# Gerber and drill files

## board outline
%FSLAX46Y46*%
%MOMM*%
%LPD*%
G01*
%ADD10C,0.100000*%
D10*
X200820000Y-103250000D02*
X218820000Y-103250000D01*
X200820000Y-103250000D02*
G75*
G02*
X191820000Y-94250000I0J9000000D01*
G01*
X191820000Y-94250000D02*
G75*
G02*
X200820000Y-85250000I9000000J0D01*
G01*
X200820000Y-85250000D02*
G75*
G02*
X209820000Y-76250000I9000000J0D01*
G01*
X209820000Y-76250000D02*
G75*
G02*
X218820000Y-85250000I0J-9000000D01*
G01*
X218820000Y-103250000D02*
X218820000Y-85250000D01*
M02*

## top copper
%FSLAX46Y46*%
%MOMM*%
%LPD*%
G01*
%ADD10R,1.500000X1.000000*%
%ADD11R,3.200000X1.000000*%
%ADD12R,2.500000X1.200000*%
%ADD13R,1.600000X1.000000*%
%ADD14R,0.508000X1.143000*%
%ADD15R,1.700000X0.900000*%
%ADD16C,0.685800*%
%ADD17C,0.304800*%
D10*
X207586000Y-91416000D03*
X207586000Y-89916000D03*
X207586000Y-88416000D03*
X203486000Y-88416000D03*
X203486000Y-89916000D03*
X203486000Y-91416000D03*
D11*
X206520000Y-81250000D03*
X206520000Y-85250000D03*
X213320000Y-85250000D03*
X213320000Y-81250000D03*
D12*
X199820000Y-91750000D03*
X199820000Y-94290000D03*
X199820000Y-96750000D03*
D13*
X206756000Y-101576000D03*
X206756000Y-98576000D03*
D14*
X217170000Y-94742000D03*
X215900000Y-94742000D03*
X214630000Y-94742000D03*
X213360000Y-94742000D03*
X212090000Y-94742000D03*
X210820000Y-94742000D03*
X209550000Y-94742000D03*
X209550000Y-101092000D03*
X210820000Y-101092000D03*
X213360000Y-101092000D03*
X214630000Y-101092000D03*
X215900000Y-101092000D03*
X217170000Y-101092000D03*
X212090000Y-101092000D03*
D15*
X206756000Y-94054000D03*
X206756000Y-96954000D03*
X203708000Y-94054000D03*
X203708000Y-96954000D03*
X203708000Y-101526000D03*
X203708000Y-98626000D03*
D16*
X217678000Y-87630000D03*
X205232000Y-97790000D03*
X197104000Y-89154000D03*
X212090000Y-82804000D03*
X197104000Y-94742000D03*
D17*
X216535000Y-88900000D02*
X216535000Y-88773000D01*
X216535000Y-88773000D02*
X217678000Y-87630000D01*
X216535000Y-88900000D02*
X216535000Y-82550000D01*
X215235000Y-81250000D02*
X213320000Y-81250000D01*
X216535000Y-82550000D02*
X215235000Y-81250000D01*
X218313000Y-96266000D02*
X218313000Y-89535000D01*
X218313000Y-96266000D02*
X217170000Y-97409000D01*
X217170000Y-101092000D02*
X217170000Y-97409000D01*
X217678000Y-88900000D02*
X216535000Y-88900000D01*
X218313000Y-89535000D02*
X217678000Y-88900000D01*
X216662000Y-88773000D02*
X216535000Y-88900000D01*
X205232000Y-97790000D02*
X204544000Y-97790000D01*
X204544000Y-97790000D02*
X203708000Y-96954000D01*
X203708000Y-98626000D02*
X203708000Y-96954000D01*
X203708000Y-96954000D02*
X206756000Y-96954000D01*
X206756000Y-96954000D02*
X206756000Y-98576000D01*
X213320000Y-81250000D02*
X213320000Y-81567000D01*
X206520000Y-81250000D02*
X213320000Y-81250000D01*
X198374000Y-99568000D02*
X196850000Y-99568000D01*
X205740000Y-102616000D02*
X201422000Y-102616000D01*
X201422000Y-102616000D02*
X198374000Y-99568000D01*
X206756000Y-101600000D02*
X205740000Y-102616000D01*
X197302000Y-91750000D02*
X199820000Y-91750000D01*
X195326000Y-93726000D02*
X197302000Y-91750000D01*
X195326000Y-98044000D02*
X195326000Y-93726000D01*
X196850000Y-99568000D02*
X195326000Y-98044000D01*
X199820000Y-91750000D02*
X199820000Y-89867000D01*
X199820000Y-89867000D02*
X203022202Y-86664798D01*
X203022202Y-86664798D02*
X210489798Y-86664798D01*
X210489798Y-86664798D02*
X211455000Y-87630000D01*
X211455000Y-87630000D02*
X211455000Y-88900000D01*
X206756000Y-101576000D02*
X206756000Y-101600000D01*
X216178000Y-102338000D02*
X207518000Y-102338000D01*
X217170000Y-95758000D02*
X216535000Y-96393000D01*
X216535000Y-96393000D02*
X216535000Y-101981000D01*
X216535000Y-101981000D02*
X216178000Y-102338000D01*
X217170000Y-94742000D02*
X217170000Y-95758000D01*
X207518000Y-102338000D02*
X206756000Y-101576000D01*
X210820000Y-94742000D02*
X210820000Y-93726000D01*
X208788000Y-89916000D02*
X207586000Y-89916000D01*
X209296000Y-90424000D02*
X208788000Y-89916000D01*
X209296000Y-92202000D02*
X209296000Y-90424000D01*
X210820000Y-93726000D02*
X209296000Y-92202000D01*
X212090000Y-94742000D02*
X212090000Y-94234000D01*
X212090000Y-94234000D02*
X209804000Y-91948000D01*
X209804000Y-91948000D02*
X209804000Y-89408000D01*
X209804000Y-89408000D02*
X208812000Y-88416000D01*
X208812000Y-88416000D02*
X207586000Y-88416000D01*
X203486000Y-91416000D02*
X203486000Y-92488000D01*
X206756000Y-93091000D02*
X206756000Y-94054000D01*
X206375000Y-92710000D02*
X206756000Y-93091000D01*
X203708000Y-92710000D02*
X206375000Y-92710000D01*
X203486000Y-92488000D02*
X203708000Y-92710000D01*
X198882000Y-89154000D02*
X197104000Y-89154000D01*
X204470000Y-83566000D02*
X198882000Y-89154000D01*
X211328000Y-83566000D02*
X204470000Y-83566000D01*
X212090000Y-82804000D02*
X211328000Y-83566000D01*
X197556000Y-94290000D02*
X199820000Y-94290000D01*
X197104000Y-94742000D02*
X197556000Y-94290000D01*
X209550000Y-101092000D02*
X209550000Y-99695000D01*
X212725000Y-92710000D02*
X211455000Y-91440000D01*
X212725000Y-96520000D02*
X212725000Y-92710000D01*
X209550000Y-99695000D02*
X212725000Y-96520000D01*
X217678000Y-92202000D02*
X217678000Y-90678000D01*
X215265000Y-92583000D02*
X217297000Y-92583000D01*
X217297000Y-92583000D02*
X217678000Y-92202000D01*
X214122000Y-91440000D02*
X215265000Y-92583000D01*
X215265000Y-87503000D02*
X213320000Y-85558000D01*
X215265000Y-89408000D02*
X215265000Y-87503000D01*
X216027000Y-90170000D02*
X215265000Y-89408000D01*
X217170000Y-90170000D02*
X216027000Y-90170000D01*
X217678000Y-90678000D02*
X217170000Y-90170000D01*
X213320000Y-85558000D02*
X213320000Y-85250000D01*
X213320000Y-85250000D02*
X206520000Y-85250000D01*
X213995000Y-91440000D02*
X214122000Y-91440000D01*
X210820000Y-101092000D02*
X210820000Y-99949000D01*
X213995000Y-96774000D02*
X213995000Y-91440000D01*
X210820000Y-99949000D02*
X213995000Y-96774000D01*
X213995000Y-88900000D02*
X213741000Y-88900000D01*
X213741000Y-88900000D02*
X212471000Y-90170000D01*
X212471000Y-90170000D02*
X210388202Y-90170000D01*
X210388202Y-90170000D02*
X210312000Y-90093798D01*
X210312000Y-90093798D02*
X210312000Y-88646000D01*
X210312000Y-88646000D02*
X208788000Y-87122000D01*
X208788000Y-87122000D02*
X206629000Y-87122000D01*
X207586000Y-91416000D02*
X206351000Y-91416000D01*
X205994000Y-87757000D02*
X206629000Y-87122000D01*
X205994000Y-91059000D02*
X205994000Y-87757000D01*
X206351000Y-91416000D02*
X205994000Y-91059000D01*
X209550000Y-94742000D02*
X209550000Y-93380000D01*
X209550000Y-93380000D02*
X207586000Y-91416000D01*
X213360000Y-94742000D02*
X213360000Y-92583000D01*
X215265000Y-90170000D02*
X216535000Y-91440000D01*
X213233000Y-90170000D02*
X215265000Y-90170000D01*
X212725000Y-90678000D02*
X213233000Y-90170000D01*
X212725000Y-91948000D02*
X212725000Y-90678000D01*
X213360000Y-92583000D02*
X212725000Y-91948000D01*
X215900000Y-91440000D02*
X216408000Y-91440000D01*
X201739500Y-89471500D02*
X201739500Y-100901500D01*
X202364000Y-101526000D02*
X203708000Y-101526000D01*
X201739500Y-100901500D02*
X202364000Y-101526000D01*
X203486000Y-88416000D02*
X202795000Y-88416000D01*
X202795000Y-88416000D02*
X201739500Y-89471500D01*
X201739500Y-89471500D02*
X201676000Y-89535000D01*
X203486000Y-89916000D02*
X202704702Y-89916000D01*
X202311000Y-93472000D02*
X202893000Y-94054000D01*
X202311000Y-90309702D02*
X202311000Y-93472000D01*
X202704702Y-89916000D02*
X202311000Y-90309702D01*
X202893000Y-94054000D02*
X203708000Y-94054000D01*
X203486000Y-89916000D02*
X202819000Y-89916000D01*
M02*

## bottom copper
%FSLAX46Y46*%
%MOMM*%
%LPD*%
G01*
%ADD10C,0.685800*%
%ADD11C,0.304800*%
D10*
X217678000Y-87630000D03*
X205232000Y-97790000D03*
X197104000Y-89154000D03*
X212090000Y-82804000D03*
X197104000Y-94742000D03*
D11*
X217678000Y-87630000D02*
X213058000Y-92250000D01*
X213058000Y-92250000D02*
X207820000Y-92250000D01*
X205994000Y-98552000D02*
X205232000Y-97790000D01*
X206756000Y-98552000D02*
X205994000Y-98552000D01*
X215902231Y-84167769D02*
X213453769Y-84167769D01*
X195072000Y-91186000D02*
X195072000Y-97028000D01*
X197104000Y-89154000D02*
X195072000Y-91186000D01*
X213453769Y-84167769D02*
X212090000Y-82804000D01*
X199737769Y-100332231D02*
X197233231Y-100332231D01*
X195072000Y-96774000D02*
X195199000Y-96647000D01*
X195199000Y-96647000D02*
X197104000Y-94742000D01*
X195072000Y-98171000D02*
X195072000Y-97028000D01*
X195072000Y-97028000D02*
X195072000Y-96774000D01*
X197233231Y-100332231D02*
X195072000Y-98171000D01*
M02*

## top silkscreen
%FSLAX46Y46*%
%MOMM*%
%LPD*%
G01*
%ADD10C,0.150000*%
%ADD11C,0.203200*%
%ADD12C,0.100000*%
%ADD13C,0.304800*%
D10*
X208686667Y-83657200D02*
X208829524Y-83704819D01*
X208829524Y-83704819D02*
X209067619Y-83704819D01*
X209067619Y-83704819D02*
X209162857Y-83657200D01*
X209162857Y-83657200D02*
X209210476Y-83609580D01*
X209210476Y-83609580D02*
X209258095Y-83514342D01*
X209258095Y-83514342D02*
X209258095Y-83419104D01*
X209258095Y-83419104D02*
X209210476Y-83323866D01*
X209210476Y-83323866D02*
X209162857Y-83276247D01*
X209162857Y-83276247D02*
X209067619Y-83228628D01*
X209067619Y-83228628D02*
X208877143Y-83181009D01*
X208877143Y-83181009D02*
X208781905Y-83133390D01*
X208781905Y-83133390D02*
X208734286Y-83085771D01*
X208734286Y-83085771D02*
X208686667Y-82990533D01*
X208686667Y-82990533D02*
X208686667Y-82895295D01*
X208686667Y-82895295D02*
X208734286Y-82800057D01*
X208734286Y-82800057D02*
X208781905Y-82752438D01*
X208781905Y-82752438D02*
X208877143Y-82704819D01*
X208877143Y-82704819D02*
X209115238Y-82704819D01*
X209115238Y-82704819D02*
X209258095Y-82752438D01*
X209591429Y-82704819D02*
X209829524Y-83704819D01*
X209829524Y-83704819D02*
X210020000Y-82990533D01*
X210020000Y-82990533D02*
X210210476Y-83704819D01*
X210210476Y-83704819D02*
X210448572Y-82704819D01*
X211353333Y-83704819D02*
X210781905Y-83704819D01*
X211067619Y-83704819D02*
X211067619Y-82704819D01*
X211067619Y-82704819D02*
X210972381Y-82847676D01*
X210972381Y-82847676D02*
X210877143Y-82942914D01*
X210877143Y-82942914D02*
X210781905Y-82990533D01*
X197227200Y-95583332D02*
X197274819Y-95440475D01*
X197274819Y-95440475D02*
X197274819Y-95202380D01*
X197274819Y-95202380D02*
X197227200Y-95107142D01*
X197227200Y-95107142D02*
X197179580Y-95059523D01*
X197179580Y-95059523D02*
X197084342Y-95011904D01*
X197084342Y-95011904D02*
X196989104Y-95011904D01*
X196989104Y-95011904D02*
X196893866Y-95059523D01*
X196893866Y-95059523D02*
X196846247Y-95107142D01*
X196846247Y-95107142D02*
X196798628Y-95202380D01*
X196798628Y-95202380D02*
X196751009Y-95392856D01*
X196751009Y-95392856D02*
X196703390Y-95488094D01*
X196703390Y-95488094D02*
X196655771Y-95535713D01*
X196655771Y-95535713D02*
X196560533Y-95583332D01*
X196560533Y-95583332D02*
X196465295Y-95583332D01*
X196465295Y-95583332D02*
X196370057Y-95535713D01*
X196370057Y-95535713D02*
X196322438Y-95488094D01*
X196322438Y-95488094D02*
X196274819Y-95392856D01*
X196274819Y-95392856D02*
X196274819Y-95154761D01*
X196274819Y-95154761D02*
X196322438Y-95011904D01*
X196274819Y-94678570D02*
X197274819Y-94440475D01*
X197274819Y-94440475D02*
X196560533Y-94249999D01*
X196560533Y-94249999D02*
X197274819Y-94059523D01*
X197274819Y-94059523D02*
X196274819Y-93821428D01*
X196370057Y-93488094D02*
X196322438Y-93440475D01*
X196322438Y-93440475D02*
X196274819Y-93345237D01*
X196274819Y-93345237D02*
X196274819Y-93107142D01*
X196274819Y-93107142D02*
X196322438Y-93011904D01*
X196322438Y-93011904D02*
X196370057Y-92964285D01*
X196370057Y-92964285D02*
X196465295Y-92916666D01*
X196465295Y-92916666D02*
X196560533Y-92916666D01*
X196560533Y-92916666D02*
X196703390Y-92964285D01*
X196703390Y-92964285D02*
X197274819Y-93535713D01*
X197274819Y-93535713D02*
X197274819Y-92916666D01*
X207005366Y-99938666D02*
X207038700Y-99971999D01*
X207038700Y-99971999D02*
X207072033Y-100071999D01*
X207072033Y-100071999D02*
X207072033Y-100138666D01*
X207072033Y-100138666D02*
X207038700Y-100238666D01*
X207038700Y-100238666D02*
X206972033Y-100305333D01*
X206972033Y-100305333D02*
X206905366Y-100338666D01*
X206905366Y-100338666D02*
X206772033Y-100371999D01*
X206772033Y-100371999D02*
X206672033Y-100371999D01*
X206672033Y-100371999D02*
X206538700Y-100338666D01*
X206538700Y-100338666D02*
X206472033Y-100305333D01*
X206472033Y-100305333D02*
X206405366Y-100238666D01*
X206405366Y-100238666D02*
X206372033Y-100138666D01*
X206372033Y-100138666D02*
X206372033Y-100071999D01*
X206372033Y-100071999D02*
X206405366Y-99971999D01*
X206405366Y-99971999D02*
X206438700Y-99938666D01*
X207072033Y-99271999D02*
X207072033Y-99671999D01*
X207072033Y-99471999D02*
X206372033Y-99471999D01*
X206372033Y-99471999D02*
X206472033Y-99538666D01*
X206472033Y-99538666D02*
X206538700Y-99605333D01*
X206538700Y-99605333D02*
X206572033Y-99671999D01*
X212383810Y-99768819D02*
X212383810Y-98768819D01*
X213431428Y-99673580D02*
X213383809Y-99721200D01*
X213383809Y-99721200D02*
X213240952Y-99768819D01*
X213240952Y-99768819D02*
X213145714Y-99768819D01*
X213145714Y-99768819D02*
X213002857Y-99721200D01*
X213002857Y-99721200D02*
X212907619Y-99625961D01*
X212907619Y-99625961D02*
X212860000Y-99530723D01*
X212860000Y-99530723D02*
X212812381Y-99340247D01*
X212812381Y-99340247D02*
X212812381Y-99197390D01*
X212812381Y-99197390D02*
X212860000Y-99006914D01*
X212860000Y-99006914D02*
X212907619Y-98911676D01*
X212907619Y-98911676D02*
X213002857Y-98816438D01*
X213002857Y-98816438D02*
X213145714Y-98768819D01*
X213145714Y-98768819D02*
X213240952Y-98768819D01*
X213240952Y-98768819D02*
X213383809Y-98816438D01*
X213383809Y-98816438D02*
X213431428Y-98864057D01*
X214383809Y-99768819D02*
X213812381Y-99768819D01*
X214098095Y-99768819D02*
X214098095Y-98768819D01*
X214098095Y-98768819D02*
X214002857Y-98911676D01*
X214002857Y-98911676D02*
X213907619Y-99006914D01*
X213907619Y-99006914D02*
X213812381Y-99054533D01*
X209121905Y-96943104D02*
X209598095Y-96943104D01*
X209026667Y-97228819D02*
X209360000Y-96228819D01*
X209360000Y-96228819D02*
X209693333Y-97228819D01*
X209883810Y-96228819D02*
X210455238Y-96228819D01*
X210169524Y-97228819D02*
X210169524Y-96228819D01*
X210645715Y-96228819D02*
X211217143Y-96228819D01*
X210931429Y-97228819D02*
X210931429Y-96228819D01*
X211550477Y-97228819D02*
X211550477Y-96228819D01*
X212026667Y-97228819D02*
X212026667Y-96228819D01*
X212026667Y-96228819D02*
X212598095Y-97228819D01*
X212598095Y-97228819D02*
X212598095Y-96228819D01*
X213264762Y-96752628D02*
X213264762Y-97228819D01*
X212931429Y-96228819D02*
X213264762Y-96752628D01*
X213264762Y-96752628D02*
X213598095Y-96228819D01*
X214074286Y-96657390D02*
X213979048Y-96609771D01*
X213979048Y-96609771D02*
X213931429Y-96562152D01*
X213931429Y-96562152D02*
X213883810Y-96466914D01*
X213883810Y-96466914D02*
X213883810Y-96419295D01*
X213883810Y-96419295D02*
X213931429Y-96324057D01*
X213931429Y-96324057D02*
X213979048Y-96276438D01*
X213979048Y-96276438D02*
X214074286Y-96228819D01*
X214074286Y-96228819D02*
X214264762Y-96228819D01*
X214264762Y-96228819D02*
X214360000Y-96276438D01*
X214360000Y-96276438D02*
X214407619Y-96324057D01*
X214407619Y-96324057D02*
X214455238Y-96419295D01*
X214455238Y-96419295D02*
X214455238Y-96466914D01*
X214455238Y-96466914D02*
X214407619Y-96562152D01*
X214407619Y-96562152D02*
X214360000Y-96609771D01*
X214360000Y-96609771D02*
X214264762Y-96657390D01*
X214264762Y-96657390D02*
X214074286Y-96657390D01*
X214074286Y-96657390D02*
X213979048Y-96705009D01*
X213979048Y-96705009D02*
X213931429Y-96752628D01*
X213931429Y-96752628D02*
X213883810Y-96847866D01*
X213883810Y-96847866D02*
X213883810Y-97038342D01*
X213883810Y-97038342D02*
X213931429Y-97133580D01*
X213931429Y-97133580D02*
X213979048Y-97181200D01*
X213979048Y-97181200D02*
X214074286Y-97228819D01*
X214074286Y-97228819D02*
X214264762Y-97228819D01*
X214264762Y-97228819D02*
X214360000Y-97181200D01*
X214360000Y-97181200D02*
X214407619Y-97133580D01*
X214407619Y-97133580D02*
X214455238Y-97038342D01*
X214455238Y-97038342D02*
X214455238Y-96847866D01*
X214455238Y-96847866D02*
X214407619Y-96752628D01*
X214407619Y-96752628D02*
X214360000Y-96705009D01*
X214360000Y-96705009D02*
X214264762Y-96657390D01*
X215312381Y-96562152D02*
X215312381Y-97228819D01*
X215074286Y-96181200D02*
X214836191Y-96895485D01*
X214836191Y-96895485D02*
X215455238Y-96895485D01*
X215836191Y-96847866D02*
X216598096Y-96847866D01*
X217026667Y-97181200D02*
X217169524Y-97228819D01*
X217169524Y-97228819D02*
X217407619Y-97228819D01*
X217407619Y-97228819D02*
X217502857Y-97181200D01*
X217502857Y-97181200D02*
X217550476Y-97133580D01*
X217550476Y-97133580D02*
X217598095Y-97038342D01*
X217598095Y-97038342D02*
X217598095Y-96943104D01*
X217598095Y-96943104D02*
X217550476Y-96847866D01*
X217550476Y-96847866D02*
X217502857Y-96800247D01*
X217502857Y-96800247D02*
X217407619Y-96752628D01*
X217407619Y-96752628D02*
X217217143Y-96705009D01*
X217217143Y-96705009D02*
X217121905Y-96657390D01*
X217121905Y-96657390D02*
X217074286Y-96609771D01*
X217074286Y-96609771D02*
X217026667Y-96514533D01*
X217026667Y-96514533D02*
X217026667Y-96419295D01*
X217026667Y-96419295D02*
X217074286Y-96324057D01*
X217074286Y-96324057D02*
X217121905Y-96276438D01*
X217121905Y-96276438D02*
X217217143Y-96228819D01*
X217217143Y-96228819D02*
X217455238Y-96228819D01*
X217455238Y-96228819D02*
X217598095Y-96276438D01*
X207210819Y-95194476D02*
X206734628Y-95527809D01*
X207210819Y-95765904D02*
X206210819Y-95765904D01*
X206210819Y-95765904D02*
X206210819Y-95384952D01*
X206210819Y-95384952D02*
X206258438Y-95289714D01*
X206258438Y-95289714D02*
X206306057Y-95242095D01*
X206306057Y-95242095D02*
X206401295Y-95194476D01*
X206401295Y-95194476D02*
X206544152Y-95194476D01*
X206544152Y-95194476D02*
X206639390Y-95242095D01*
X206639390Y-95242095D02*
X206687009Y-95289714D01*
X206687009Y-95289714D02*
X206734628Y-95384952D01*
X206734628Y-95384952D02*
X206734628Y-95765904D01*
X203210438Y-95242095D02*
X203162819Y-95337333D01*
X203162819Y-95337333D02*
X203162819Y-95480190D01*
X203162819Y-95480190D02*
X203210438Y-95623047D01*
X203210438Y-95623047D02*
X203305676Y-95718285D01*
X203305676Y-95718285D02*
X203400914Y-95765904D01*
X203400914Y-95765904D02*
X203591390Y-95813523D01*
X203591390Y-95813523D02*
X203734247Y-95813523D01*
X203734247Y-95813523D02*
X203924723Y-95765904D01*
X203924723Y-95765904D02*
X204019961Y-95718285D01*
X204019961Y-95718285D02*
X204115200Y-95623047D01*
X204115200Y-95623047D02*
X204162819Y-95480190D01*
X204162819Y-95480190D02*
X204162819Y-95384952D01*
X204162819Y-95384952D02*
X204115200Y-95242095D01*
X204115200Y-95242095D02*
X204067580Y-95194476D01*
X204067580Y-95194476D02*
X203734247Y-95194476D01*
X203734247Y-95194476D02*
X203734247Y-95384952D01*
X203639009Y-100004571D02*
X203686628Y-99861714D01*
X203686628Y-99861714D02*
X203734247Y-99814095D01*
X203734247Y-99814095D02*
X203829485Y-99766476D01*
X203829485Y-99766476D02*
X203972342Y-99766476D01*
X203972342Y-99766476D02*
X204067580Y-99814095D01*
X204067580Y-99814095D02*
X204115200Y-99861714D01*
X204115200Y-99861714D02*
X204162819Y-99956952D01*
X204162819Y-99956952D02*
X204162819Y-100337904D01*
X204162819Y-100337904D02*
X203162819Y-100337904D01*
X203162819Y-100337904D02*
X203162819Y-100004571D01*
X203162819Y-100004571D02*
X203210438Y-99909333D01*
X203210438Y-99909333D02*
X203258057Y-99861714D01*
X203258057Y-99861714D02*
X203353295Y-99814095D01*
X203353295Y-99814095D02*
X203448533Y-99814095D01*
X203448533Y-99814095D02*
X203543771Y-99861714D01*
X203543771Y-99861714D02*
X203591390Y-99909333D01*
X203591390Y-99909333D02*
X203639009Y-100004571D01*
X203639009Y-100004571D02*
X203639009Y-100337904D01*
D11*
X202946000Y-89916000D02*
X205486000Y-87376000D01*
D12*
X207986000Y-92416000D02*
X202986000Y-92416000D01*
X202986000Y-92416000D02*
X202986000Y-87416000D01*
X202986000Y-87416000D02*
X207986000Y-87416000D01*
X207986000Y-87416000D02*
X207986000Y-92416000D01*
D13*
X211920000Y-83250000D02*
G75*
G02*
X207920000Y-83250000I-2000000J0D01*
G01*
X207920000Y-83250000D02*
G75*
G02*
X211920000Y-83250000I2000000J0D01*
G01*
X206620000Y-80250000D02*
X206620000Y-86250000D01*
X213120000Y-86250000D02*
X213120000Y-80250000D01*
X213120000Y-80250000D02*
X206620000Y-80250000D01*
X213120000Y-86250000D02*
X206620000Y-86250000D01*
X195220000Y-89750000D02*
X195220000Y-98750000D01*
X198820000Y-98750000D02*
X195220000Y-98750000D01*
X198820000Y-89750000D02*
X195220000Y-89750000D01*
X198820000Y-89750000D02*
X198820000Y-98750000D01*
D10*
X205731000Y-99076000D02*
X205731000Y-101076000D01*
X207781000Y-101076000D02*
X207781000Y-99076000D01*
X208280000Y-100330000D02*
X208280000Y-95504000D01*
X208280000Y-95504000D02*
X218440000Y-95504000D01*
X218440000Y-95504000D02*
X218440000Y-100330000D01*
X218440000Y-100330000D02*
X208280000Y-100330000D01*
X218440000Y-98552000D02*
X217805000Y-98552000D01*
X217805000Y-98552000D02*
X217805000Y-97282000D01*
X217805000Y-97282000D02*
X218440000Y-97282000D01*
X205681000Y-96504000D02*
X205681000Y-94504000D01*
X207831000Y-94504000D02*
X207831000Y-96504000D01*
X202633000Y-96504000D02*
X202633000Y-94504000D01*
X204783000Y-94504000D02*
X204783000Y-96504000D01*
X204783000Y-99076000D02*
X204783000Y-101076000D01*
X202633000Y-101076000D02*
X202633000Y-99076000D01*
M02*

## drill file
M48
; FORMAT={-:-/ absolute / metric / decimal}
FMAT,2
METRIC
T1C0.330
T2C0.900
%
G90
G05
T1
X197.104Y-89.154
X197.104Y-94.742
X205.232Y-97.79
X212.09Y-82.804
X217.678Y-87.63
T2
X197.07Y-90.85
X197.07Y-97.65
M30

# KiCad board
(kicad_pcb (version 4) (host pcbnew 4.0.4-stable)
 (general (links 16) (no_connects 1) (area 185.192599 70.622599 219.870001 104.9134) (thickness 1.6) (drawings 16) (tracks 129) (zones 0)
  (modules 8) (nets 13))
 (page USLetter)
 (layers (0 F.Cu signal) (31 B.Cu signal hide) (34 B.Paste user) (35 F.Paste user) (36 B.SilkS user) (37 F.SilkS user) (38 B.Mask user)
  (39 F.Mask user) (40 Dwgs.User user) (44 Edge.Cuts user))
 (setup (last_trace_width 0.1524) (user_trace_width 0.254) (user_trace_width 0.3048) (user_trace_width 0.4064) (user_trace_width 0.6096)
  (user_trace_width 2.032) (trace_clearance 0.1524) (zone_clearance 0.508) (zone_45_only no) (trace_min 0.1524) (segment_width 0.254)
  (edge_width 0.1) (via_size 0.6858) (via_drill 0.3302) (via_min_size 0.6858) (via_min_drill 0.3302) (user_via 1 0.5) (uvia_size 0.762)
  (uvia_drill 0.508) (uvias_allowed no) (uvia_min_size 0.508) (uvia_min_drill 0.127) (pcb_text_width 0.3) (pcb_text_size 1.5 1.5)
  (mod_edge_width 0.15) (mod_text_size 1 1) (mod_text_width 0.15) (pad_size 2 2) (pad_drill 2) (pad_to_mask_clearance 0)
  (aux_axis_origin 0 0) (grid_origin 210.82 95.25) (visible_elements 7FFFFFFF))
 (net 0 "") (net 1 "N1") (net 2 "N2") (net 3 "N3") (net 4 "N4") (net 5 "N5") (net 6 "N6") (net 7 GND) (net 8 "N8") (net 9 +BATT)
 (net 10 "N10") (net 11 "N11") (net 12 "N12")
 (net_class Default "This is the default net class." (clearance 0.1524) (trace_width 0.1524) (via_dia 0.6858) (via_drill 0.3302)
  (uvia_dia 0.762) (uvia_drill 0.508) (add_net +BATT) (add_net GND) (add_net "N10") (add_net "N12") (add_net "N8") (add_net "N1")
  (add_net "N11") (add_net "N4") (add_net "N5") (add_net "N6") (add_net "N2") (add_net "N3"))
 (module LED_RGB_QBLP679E (layer F.Cu) (at 205.486 89.916 180)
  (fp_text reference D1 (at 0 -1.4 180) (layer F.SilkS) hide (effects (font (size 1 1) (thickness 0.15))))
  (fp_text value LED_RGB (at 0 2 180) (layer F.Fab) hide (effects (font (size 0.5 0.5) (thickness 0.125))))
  (fp_line (start 2.54 0) (end 0 2.54) (layer F.SilkS) (width 0.2032))
  (fp_line (start -2.5 -2.5) (end 2.5 -2.5) (layer F.SilkS) (width 0.1))
  (fp_line (start 2.5 -2.5) (end 2.5 2.5) (layer F.SilkS) (width 0.1))
  (fp_line (start 2.5 2.5) (end -2.5 2.5) (layer F.SilkS) (width 0.1))
  (fp_line (start -2.5 2.5) (end -2.5 -2.5) (layer F.SilkS) (width 0.1))
  (pad 4 smd rect (at -2.1 -1.5 270) (size 1 1.5) (layers F.Cu F.Paste F.Mask) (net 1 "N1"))
  (pad 5 smd rect (at -2.1 0 270) (size 1 1.5) (layers F.Cu F.Paste F.Mask) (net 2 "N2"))
  (pad 6 smd rect (at -2.1 1.5 270) (size 1 1.5) (layers F.Cu F.Paste F.Mask) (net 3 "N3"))
  (pad 1 smd rect (at 2 1.5 270) (size 1 1.5) (layers F.Cu F.Paste F.Mask) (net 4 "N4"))
  (pad 2 smd rect (at 2 0 270) (size 1 1.5) (layers F.Cu F.Paste F.Mask) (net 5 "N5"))
  (pad 3 smd rect (at 2 -1.5 270) (size 1 1.5) (layers F.Cu F.Paste F.Mask) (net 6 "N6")))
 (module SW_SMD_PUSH (layer F.Cu) (at 213.32 85.25 180)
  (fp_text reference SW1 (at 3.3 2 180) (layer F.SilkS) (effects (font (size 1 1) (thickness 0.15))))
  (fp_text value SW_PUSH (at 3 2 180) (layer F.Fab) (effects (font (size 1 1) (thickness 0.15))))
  (fp_circle (center 3.4 2) (end 3.4 0) (layer F.SilkS) (width 0.3048))
  (fp_line (start 6.7 5) (end 6.7 -1) (layer F.SilkS) (width 0.3048))
  (fp_line (start 0.2 -1) (end 0.2 5) (layer F.SilkS) (width 0.3048))
  (fp_line (start 0.2 5) (end 6.7 5) (layer F.SilkS) (width 0.3048))
  (fp_line (start 0.2 -1) (end 6.7 -1) (layer F.SilkS) (width 0.3048))
  (pad 2 smd rect (at 6.8 4 180) (size 3.2 1) (layers F.Cu F.Paste F.Mask) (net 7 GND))
  (pad 1 smd rect (at 6.8 0 180) (size 3.2 1) (layers F.Cu F.Paste F.Mask) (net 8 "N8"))
  (pad 1 smd rect (at 0 0 180) (size 3.2 1) (layers F.Cu F.Paste F.Mask) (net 8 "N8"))
  (pad 2 smd rect (at 0 4 180) (size 3.2 1) (layers F.Cu F.Paste F.Mask) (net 7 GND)))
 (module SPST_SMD (layer F.Cu) (at 199.82 94.25 270)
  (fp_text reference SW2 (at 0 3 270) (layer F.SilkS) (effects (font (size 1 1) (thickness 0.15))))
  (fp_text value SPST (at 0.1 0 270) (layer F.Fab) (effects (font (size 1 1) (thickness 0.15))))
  (fp_line (start -4.5 4.6) (end 4.5 4.6) (layer F.SilkS) (width 0.3048))
  (fp_line (start 4.5 1) (end 4.5 4.6) (layer F.SilkS) (width 0.3048))
  (fp_line (start -4.5 1) (end -4.5 4.6) (layer F.SilkS) (width 0.3048))
  (fp_line (start -4.5 1) (end 4.5 1) (layer F.SilkS) (width 0.3048))
  (pad "" np_thru_hole circle (at 3.4 2.75 270) (size 0.9 0.9) (drill 0.9) (layers *.Cu *.Mask))
  (pad 1 smd rect (at -2.5 0 270) (size 1.2 2.5) (layers F.Cu F.Paste F.Mask) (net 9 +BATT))
  (pad 2 smd rect (at 0.04 0 270) (size 1.2 2.5) (layers F.Cu F.Paste F.Mask) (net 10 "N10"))
  (pad 3 smd rect (at 2.5 0 270) (size 1.2 2.5) (layers F.Cu F.Paste F.Mask))
  (pad "" np_thru_hole circle (at -3.4 2.75 270) (size 0.9 0.9) (drill 0.9) (layers *.Cu *.Mask)))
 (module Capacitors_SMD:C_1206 (layer F.Cu) (at 206.756 100.076 90)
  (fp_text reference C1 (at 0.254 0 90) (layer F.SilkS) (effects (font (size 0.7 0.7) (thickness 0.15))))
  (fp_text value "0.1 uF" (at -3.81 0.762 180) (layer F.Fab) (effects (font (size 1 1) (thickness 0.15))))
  (fp_line (start 1 -1.025) (end -1 -1.025) (layer F.SilkS) (width 0.15))
  (fp_line (start -1 1.025) (end 1 1.025) (layer F.SilkS) (width 0.15))
  (pad 1 smd rect (at -1.5 0 90) (size 1 1.6) (layers F.Cu F.Paste F.Mask) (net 9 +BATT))
  (pad 2 smd rect (at 1.5 0 90) (size 1 1.6) (layers F.Cu F.Paste F.Mask) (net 7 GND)))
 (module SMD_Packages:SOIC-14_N (layer F.Cu) (at 213.36 98.044 180)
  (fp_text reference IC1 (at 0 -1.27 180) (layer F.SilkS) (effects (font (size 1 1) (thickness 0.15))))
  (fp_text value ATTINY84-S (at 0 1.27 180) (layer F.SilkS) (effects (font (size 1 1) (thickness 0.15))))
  (fp_line (start 5.08 -2.286) (end 5.08 2.54) (layer F.SilkS) (width 0.15))
  (fp_line (start 5.08 2.54) (end -5.08 2.54) (layer F.SilkS) (width 0.15))
  (fp_line (start -5.08 2.54) (end -5.08 -2.286) (layer F.SilkS) (width 0.15))
  (fp_line (start -5.08 -2.286) (end 5.08 -2.286) (layer F.SilkS) (width 0.15))
  (fp_line (start -5.08 -0.508) (end -4.445 -0.508) (layer F.SilkS) (width 0.15))
  (fp_line (start -4.445 -0.508) (end -4.445 0.762) (layer F.SilkS) (width 0.15))
  (fp_line (start -4.445 0.762) (end -5.08 0.762) (layer F.SilkS) (width 0.15))
  (pad 1 smd rect (at -3.81 3.302 180) (size 0.508 1.143) (layers F.Cu F.Paste F.Mask) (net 9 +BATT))
  (pad 2 smd rect (at -2.54 3.302 180) (size 0.508 1.143) (layers F.Cu F.Paste F.Mask))
  (pad 3 smd rect (at -1.27 3.302 180) (size 0.508 1.143) (layers F.Cu F.Paste F.Mask))
  (pad 4 smd rect (at 0 3.302 180) (size 0.508 1.143) (layers F.Cu F.Paste F.Mask) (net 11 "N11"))
  (pad 5 smd rect (at 1.27 3.302 180) (size 0.508 1.143) (layers F.Cu F.Paste F.Mask) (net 3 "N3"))
  (pad 6 smd rect (at 2.54 3.302 180) (size 0.508 1.143) (layers F.Cu F.Paste F.Mask) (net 2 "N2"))
  (pad 7 smd rect (at 3.81 3.302 180) (size 0.508 1.143) (layers F.Cu F.Paste F.Mask) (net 1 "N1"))
  (pad 8 smd rect (at 3.81 -3.048 180) (size 0.508 1.143) (layers F.Cu F.Paste F.Mask) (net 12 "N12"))
  (pad 9 smd rect (at 2.54 -3.048 180) (size 0.508 1.143) (layers F.Cu F.Paste F.Mask) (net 8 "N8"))
  (pad 11 smd rect (at 0 -3.048 180) (size 0.508 1.143) (layers F.Cu F.Paste F.Mask))
  (pad 12 smd rect (at -1.27 -3.048 180) (size 0.508 1.143) (layers F.Cu F.Paste F.Mask))
  (pad 13 smd rect (at -2.54 -3.048 180) (size 0.508 1.143) (layers F.Cu F.Paste F.Mask))
  (pad 14 smd rect (at -3.81 -3.048 180) (size 0.508 1.143) (layers F.Cu F.Paste F.Mask) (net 7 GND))
  (pad 10 smd rect (at 1.27 -3.048 180) (size 0.508 1.143) (layers F.Cu F.Paste F.Mask)))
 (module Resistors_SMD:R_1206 (layer F.Cu) (at 206.756 95.504 270)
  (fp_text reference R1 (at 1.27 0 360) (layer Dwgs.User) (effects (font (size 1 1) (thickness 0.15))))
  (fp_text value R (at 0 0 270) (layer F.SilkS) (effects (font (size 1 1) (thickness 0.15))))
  (fp_line (start 1 1.075) (end -1 1.075) (layer F.SilkS) (width 0.15))
  (fp_line (start -1 -1.075) (end 1 -1.075) (layer F.SilkS) (width 0.15))
  (pad 1 smd rect (at -1.45 0 270) (size 0.9 1.7) (layers F.Cu F.Paste F.Mask) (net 6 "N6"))
  (pad 2 smd rect (at 1.45 0 270) (size 0.9 1.7) (layers F.Cu F.Paste F.Mask) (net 7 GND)))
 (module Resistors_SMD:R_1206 (layer F.Cu) (at 203.708 95.504 270)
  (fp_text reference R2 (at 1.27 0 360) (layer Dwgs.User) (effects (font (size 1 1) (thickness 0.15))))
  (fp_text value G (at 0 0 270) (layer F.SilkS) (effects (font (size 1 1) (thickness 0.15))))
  (fp_line (start 1 1.075) (end -1 1.075) (layer F.SilkS) (width 0.15))
  (fp_line (start -1 -1.075) (end 1 -1.075) (layer F.SilkS) (width 0.15))
  (pad 1 smd rect (at -1.45 0 270) (size 0.9 1.7) (layers F.Cu F.Paste F.Mask) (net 5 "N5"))
  (pad 2 smd rect (at 1.45 0 270) (size 0.9 1.7) (layers F.Cu F.Paste F.Mask) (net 7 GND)))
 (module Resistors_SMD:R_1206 (layer F.Cu) (at 203.708 100.076 90)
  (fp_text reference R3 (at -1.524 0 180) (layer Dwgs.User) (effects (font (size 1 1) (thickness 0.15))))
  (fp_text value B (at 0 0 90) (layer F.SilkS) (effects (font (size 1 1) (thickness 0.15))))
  (fp_line (start 1 1.075) (end -1 1.075) (layer F.SilkS) (width 0.15))
  (fp_line (start -1 -1.075) (end 1 -1.075) (layer F.SilkS) (width 0.15))
  (pad 1 smd rect (at -1.45 0 90) (size 0.9 1.7) (layers F.Cu F.Paste F.Mask) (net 4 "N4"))
  (pad 2 smd rect (at 1.45 0 90) (size 0.9 1.7) (layers F.Cu F.Paste F.Mask) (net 7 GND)))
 (gr_line (start 200.82 103.25) (end 218.82 103.25) (angle 90) (layer Edge.Cuts) (width 0.1))
 (gr_arc (start 200.82 94.25) (end 200.82 103.25) (angle 90) (layer Edge.Cuts) (width 0.1))
 (gr_arc (start 200.82 94.25) (end 191.82 94.25) (angle 90) (layer Edge.Cuts) (width 0.1))
 (gr_arc (start 209.82 85.25) (end 200.82 85.25) (angle 90) (layer Edge.Cuts) (width 0.1))
 (gr_arc (start 209.82 85.25) (end 209.82 76.25) (angle 90) (layer Edge.Cuts) (width 0.1))
 (gr_line (start 218.82 103.25) (end 218.82 85.25) (angle 90) (layer Edge.Cuts) (width 0.1))
 (segment (start 216.535 88.9) (end 216.535 88.773) (width 0.3048) (layer F.Cu) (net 7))
 (segment (start 216.535 88.773) (end 217.678 87.63) (width 0.3048) (layer F.Cu) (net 7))
 (segment (start 217.678 87.63) (end 213.058 92.25) (width 0.3048) (layer B.Cu) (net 7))
 (via (at 217.678 87.63) (size 0.6858) (drill 0.3302) (layers F.Cu B.Cu) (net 7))
 (segment (start 213.058 92.25) (end 207.82 92.25) (width 0.3048) (layer B.Cu) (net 7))
 (segment (start 216.535 88.9) (end 216.535 82.55) (width 0.3048) (layer F.Cu) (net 7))
 (segment (start 215.235 81.25) (end 213.32 81.25) (width 0.3048) (layer F.Cu) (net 7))
 (segment (start 216.535 82.55) (end 215.235 81.25) (width 0.3048) (layer F.Cu) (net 7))
 (segment (start 218.313 96.266) (end 218.313 89.535) (width 0.3048) (layer F.Cu) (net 7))
 (segment (start 218.313 96.266) (end 217.17 97.409) (width 0.3048) (layer F.Cu) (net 7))
 (segment (start 217.17 101.092) (end 217.17 97.409) (width 0.3048) (layer F.Cu) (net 7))
 (segment (start 217.678 88.9) (end 216.535 88.9) (width 0.3048) (layer F.Cu) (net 7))
 (segment (start 218.313 89.535) (end 217.678 88.9) (width 0.3048) (layer F.Cu) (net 7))
 (segment (start 216.662 88.773) (end 216.535 88.9) (width 0.3048) (layer F.Cu) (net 7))
 (segment (start 205.232 97.79) (end 204.544 97.79) (width 0.3048) (layer F.Cu) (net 7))
 (segment (start 205.994 98.552) (end 205.232 97.79) (width 0.3048) (layer B.Cu) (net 7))
 (via (at 205.232 97.79) (size 0.6858) (drill 0.3302) (layers F.Cu B.Cu) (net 7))
 (segment (start 204.544 97.79) (end 203.708 96.954) (width 0.3048) (layer F.Cu) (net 7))
 (segment (start 206.756 98.552) (end 205.994 98.552) (width 0.3048) (layer B.Cu) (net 7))
 (segment (start 203.708 98.626) (end 203.708 96.954) (width 0.3048) (layer F.Cu) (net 7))
 (segment (start 203.708 96.954) (end 206.756 96.954) (width 0.3048) (layer F.Cu) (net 7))
 (segment (start 206.756 96.954) (end 206.756 98.576) (width 0.3048) (layer F.Cu) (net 7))
 (segment (start 213.32 81.25) (end 213.32 81.567) (width 0.3048) (layer F.Cu) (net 7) (status 30))
 (segment (start 206.52 81.25) (end 213.32 81.25) (width 0.3048) (layer F.Cu) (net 7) (status 30))
 (segment (start 198.374 99.568) (end 196.85 99.568) (width 0.3048) (layer F.Cu) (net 9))
 (segment (start 205.74 102.616) (end 201.422 102.616) (width 0.3048) (layer F.Cu) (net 9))
 (segment (start 201.422 102.616) (end 198.374 99.568) (width 0.3048) (layer F.Cu) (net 9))
 (segment (start 206.756 101.6) (end 205.74 102.616) (width 0.3048) (layer F.Cu) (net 9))
 (segment (start 197.302 91.75) (end 199.82 91.75) (width 0.3048) (layer F.Cu) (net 9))
 (segment (start 195.326 93.726) (end 197.302 91.75) (width 0.3048) (layer F.Cu) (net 9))
 (segment (start 195.326 98.044) (end 195.326 93.726) (width 0.3048) (layer F.Cu) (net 9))
 (segment (start 196.85 99.568) (end 195.326 98.044) (width 0.3048) (layer F.Cu) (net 9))
 (segment (start 199.82 91.75) (end 199.82 89.867) (width 0.3048) (layer F.Cu) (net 9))
 (segment (start 199.82 89.867) (end 203.022202 86.664798) (width 0.3048) (layer F.Cu) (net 9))
 (segment (start 203.022202 86.664798) (end 210.489798 86.664798) (width 0.3048) (layer F.Cu) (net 9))
 (segment (start 210.489798 86.664798) (end 211.455 87.63) (width 0.3048) (layer F.Cu) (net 9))
 (segment (start 211.455 87.63) (end 211.455 88.9) (width 0.3048) (layer F.Cu) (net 9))
 (segment (start 206.756 101.576) (end 206.756 101.6) (width 0.3048) (layer F.Cu) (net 9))
 (segment (start 216.178 102.338) (end 207.518 102.338) (width 0.3048) (layer F.Cu) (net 9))
 (segment (start 217.17 95.758) (end 216.535 96.393) (width 0.3048) (layer F.Cu) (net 9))
 (segment (start 216.535 96.393) (end 216.535 101.981) (width 0.3048) (layer F.Cu) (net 9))
 (segment (start 216.535 101.981) (end 216.178 102.338) (width 0.3048) (layer F.Cu) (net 9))
 (segment (start 217.17 94.742) (end 217.17 95.758) (width 0.3048) (layer F.Cu) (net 9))
 (segment (start 207.518 102.338) (end 206.756 101.576) (width 0.3048) (layer F.Cu) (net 9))
 (segment (start 210.82 94.742) (end 210.82 93.726) (width 0.3048) (layer F.Cu) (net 2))
 (segment (start 208.788 89.916) (end 207.586 89.916) (width 0.3048) (layer F.Cu) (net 2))
 (segment (start 209.296 90.424) (end 208.788 89.916) (width 0.3048) (layer F.Cu) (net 2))
 (segment (start 209.296 92.202) (end 209.296 90.424) (width 0.3048) (layer F.Cu) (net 2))
 (segment (start 210.82 93.726) (end 209.296 92.202) (width 0.3048) (layer F.Cu) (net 2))
 (segment (start 212.09 94.742) (end 212.09 94.234) (width 0.3048) (layer F.Cu) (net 3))
 (segment (start 212.09 94.234) (end 209.804 91.948) (width 0.3048) (layer F.Cu) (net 3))
 (segment (start 209.804 91.948) (end 209.804 89.408) (width 0.3048) (layer F.Cu) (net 3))
 (segment (start 209.804 89.408) (end 208.812 88.416) (width 0.3048) (layer F.Cu) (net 3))
 (segment (start 208.812 88.416) (end 207.586 88.416) (width 0.3048) (layer F.Cu) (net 3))
 (segment (start 203.486 91.416) (end 203.486 92.488) (width 0.3048) (layer F.Cu) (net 6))
 (segment (start 206.756 93.091) (end 206.756 94.054) (width 0.3048) (layer F.Cu) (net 6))
 (segment (start 206.375 92.71) (end 206.756 93.091) (width 0.3048) (layer F.Cu) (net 6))
 (segment (start 203.708 92.71) (end 206.375 92.71) (width 0.3048) (layer F.Cu) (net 6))
 (segment (start 203.486 92.488) (end 203.708 92.71) (width 0.3048) (layer F.Cu) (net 6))
 (segment (start 215.902231 84.167769) (end 213.453769 84.167769) (width 0.3048) (layer B.Cu) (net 10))
 (segment (start 195.072 91.186) (end 195.072 97.028) (width 0.3048) (layer B.Cu) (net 10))
 (segment (start 197.104 89.154) (end 195.072 91.186) (width 0.3048) (layer B.Cu) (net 10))
 (via (at 197.104 89.154) (size 0.6858) (drill 0.3302) (layers F.Cu B.Cu) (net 10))
 (segment (start 198.882 89.154) (end 197.104 89.154) (width 0.3048) (layer F.Cu) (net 10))
 (segment (start 204.47 83.566) (end 198.882 89.154) (width 0.3048) (layer F.Cu) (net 10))
 (segment (start 211.328 83.566) (end 204.47 83.566) (width 0.3048) (layer F.Cu) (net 10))
 (segment (start 212.09 82.804) (end 211.328 83.566) (width 0.3048) (layer F.Cu) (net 10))
 (via (at 212.09 82.804) (size 0.6858) (drill 0.3302) (layers F.Cu B.Cu) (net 10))
 (segment (start 213.453769 84.167769) (end 212.09 82.804) (width 0.3048) (layer B.Cu) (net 10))
 (segment (start 199.737769 100.332231) (end 197.233231 100.332231) (width 0.3048) (layer B.Cu) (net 10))
 (segment (start 197.556 94.29) (end 199.82 94.29) (width 0.3048) (layer F.Cu) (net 10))
 (segment (start 197.104 94.742) (end 197.556 94.29) (width 0.3048) (layer F.Cu) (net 10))
 (via (at 197.104 94.742) (size 0.6858) (drill 0.3302) (layers F.Cu B.Cu) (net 10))
 (segment (start 195.072 96.774) (end 195.199 96.647) (width 0.3048) (layer B.Cu) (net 10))
 (segment (start 195.199 96.647) (end 197.104 94.742) (width 0.3048) (layer B.Cu) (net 10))
 (segment (start 195.072 98.171) (end 195.072 97.028) (width 0.3048) (layer B.Cu) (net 10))
 (segment (start 195.072 97.028) (end 195.072 96.774) (width 0.3048) (layer B.Cu) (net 10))
 (segment (start 197.233231 100.332231) (end 195.072 98.171) (width 0.3048) (layer B.Cu) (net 10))
 (segment (start 209.55 101.092) (end 209.55 99.695) (width 0.3048) (layer F.Cu) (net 12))
 (segment (start 212.725 92.71) (end 211.455 91.44) (width 0.3048) (layer F.Cu) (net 12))
 (segment (start 212.725 96.52) (end 212.725 92.71) (width 0.3048) (layer F.Cu) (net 12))
 (segment (start 209.55 99.695) (end 212.725 96.52) (width 0.3048) (layer F.Cu) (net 12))
 (segment (start 217.678 92.202) (end 217.678 90.678) (width 0.3048) (layer F.Cu) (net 8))
 (segment (start 215.265 92.583) (end 217.297 92.583) (width 0.3048) (layer F.Cu) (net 8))
 (segment (start 217.297 92.583) (end 217.678 92.202) (width 0.3048) (layer F.Cu) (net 8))
 (segment (start 214.122 91.44) (end 215.265 92.583) (width 0.3048) (layer F.Cu) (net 8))
 (segment (start 215.265 87.503) (end 213.32 85.558) (width 0.3048) (layer F.Cu) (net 8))
 (segment (start 215.265 89.408) (end 215.265 87.503) (width 0.3048) (layer F.Cu) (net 8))
 (segment (start 216.027 90.17) (end 215.265 89.408) (width 0.3048) (layer F.Cu) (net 8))
 (segment (start 217.17 90.17) (end 216.027 90.17) (width 0.3048) (layer F.Cu) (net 8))
 (segment (start 217.678 90.678) (end 217.17 90.17) (width 0.3048) (layer F.Cu) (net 8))
 (segment (start 213.32 85.558) (end 213.32 85.25) (width 0.3048) (layer F.Cu) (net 8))
 (segment (start 213.32 85.25) (end 206.52 85.25) (width 0.3048) (layer F.Cu) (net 8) (status 30))
 (segment (start 213.995 91.44) (end 214.122 91.44) (width 0.3048) (layer F.Cu) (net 8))
 (segment (start 210.82 101.092) (end 210.82 99.949) (width 0.3048) (layer F.Cu) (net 8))
 (segment (start 213.995 96.774) (end 213.995 91.44) (width 0.3048) (layer F.Cu) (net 8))
 (segment (start 210.82 99.949) (end 213.995 96.774) (width 0.3048) (layer F.Cu) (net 8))
 (segment (start 213.995 88.9) (end 213.741 88.9) (width 0.3048) (layer F.Cu) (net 1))
 (segment (start 213.741 88.9) (end 212.471 90.17) (width 0.3048) (layer F.Cu) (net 1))
 (segment (start 212.471 90.17) (end 210.388202 90.17) (width 0.3048) (layer F.Cu) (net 1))
 (segment (start 210.388202 90.17) (end 210.312 90.093798) (width 0.3048) (layer F.Cu) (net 1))
 (segment (start 210.312 90.093798) (end 210.312 88.646) (width 0.3048) (layer F.Cu) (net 1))
 (segment (start 210.312 88.646) (end 208.788 87.122) (width 0.3048) (layer F.Cu) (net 1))
 (segment (start 208.788 87.122) (end 206.629 87.122) (width 0.3048) (layer F.Cu) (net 1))
 (segment (start 207.586 91.416) (end 206.351 91.416) (width 0.3048) (layer F.Cu) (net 1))
 (segment (start 205.994 87.757) (end 206.629 87.122) (width 0.3048) (layer F.Cu) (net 1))
 (segment (start 205.994 91.059) (end 205.994 87.757) (width 0.3048) (layer F.Cu) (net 1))
 (segment (start 206.351 91.416) (end 205.994 91.059) (width 0.3048) (layer F.Cu) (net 1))
 (segment (start 209.55 94.742) (end 209.55 93.38) (width 0.3048) (layer F.Cu) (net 1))
 (segment (start 209.55 93.38) (end 207.586 91.416) (width 0.3048) (layer F.Cu) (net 1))
 (segment (start 213.36 94.742) (end 213.36 92.583) (width 0.3048) (layer F.Cu) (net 11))
 (segment (start 215.265 90.17) (end 216.535 91.44) (width 0.3048) (layer F.Cu) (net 11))
 (segment (start 213.233 90.17) (end 215.265 90.17) (width 0.3048) (layer F.Cu) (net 11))
 (segment (start 212.725 90.678) (end 213.233 90.17) (width 0.3048) (layer F.Cu) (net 11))
 (segment (start 212.725 91.948) (end 212.725 90.678) (width 0.3048) (layer F.Cu) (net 11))
 (segment (start 213.36 92.583) (end 212.725 91.948) (width 0.3048) (layer F.Cu) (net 11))
 (segment (start 215.9 91.44) (end 216.408 91.44) (width 0.3048) (layer F.Cu) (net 11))
 (segment (start 201.7395 89.4715) (end 201.7395 100.9015) (width 0.3048) (layer F.Cu) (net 4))
 (segment (start 202.364 101.526) (end 203.708 101.526) (width 0.3048) (layer F.Cu) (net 4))
 (segment (start 201.7395 100.9015) (end 202.364 101.526) (width 0.3048) (layer F.Cu) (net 4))
 (segment (start 203.486 88.416) (end 202.795 88.416) (width 0.3048) (layer F.Cu) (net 4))
 (segment (start 202.795 88.416) (end 201.7395 89.4715) (width 0.3048) (layer F.Cu) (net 4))
 (segment (start 201.7395 89.4715) (end 201.676 89.535) (width 0.3048) (layer F.Cu) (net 4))
 (segment (start 203.486 89.916) (end 202.704702 89.916) (width 0.3048) (layer F.Cu) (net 5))
 (segment (start 202.311 93.472) (end 202.893 94.054) (width 0.3048) (layer F.Cu) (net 5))
 (segment (start 202.311 90.309702) (end 202.311 93.472) (width 0.3048) (layer F.Cu) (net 5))
 (segment (start 202.704702 89.916) (end 202.311 90.309702) (width 0.3048) (layer F.Cu) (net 5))
 (segment (start 202.893 94.054) (end 203.708 94.054) (width 0.3048) (layer F.Cu) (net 5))
 (segment (start 203.486 89.916) (end 202.819 89.916) (width 0.3048) (layer F.Cu) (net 5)))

